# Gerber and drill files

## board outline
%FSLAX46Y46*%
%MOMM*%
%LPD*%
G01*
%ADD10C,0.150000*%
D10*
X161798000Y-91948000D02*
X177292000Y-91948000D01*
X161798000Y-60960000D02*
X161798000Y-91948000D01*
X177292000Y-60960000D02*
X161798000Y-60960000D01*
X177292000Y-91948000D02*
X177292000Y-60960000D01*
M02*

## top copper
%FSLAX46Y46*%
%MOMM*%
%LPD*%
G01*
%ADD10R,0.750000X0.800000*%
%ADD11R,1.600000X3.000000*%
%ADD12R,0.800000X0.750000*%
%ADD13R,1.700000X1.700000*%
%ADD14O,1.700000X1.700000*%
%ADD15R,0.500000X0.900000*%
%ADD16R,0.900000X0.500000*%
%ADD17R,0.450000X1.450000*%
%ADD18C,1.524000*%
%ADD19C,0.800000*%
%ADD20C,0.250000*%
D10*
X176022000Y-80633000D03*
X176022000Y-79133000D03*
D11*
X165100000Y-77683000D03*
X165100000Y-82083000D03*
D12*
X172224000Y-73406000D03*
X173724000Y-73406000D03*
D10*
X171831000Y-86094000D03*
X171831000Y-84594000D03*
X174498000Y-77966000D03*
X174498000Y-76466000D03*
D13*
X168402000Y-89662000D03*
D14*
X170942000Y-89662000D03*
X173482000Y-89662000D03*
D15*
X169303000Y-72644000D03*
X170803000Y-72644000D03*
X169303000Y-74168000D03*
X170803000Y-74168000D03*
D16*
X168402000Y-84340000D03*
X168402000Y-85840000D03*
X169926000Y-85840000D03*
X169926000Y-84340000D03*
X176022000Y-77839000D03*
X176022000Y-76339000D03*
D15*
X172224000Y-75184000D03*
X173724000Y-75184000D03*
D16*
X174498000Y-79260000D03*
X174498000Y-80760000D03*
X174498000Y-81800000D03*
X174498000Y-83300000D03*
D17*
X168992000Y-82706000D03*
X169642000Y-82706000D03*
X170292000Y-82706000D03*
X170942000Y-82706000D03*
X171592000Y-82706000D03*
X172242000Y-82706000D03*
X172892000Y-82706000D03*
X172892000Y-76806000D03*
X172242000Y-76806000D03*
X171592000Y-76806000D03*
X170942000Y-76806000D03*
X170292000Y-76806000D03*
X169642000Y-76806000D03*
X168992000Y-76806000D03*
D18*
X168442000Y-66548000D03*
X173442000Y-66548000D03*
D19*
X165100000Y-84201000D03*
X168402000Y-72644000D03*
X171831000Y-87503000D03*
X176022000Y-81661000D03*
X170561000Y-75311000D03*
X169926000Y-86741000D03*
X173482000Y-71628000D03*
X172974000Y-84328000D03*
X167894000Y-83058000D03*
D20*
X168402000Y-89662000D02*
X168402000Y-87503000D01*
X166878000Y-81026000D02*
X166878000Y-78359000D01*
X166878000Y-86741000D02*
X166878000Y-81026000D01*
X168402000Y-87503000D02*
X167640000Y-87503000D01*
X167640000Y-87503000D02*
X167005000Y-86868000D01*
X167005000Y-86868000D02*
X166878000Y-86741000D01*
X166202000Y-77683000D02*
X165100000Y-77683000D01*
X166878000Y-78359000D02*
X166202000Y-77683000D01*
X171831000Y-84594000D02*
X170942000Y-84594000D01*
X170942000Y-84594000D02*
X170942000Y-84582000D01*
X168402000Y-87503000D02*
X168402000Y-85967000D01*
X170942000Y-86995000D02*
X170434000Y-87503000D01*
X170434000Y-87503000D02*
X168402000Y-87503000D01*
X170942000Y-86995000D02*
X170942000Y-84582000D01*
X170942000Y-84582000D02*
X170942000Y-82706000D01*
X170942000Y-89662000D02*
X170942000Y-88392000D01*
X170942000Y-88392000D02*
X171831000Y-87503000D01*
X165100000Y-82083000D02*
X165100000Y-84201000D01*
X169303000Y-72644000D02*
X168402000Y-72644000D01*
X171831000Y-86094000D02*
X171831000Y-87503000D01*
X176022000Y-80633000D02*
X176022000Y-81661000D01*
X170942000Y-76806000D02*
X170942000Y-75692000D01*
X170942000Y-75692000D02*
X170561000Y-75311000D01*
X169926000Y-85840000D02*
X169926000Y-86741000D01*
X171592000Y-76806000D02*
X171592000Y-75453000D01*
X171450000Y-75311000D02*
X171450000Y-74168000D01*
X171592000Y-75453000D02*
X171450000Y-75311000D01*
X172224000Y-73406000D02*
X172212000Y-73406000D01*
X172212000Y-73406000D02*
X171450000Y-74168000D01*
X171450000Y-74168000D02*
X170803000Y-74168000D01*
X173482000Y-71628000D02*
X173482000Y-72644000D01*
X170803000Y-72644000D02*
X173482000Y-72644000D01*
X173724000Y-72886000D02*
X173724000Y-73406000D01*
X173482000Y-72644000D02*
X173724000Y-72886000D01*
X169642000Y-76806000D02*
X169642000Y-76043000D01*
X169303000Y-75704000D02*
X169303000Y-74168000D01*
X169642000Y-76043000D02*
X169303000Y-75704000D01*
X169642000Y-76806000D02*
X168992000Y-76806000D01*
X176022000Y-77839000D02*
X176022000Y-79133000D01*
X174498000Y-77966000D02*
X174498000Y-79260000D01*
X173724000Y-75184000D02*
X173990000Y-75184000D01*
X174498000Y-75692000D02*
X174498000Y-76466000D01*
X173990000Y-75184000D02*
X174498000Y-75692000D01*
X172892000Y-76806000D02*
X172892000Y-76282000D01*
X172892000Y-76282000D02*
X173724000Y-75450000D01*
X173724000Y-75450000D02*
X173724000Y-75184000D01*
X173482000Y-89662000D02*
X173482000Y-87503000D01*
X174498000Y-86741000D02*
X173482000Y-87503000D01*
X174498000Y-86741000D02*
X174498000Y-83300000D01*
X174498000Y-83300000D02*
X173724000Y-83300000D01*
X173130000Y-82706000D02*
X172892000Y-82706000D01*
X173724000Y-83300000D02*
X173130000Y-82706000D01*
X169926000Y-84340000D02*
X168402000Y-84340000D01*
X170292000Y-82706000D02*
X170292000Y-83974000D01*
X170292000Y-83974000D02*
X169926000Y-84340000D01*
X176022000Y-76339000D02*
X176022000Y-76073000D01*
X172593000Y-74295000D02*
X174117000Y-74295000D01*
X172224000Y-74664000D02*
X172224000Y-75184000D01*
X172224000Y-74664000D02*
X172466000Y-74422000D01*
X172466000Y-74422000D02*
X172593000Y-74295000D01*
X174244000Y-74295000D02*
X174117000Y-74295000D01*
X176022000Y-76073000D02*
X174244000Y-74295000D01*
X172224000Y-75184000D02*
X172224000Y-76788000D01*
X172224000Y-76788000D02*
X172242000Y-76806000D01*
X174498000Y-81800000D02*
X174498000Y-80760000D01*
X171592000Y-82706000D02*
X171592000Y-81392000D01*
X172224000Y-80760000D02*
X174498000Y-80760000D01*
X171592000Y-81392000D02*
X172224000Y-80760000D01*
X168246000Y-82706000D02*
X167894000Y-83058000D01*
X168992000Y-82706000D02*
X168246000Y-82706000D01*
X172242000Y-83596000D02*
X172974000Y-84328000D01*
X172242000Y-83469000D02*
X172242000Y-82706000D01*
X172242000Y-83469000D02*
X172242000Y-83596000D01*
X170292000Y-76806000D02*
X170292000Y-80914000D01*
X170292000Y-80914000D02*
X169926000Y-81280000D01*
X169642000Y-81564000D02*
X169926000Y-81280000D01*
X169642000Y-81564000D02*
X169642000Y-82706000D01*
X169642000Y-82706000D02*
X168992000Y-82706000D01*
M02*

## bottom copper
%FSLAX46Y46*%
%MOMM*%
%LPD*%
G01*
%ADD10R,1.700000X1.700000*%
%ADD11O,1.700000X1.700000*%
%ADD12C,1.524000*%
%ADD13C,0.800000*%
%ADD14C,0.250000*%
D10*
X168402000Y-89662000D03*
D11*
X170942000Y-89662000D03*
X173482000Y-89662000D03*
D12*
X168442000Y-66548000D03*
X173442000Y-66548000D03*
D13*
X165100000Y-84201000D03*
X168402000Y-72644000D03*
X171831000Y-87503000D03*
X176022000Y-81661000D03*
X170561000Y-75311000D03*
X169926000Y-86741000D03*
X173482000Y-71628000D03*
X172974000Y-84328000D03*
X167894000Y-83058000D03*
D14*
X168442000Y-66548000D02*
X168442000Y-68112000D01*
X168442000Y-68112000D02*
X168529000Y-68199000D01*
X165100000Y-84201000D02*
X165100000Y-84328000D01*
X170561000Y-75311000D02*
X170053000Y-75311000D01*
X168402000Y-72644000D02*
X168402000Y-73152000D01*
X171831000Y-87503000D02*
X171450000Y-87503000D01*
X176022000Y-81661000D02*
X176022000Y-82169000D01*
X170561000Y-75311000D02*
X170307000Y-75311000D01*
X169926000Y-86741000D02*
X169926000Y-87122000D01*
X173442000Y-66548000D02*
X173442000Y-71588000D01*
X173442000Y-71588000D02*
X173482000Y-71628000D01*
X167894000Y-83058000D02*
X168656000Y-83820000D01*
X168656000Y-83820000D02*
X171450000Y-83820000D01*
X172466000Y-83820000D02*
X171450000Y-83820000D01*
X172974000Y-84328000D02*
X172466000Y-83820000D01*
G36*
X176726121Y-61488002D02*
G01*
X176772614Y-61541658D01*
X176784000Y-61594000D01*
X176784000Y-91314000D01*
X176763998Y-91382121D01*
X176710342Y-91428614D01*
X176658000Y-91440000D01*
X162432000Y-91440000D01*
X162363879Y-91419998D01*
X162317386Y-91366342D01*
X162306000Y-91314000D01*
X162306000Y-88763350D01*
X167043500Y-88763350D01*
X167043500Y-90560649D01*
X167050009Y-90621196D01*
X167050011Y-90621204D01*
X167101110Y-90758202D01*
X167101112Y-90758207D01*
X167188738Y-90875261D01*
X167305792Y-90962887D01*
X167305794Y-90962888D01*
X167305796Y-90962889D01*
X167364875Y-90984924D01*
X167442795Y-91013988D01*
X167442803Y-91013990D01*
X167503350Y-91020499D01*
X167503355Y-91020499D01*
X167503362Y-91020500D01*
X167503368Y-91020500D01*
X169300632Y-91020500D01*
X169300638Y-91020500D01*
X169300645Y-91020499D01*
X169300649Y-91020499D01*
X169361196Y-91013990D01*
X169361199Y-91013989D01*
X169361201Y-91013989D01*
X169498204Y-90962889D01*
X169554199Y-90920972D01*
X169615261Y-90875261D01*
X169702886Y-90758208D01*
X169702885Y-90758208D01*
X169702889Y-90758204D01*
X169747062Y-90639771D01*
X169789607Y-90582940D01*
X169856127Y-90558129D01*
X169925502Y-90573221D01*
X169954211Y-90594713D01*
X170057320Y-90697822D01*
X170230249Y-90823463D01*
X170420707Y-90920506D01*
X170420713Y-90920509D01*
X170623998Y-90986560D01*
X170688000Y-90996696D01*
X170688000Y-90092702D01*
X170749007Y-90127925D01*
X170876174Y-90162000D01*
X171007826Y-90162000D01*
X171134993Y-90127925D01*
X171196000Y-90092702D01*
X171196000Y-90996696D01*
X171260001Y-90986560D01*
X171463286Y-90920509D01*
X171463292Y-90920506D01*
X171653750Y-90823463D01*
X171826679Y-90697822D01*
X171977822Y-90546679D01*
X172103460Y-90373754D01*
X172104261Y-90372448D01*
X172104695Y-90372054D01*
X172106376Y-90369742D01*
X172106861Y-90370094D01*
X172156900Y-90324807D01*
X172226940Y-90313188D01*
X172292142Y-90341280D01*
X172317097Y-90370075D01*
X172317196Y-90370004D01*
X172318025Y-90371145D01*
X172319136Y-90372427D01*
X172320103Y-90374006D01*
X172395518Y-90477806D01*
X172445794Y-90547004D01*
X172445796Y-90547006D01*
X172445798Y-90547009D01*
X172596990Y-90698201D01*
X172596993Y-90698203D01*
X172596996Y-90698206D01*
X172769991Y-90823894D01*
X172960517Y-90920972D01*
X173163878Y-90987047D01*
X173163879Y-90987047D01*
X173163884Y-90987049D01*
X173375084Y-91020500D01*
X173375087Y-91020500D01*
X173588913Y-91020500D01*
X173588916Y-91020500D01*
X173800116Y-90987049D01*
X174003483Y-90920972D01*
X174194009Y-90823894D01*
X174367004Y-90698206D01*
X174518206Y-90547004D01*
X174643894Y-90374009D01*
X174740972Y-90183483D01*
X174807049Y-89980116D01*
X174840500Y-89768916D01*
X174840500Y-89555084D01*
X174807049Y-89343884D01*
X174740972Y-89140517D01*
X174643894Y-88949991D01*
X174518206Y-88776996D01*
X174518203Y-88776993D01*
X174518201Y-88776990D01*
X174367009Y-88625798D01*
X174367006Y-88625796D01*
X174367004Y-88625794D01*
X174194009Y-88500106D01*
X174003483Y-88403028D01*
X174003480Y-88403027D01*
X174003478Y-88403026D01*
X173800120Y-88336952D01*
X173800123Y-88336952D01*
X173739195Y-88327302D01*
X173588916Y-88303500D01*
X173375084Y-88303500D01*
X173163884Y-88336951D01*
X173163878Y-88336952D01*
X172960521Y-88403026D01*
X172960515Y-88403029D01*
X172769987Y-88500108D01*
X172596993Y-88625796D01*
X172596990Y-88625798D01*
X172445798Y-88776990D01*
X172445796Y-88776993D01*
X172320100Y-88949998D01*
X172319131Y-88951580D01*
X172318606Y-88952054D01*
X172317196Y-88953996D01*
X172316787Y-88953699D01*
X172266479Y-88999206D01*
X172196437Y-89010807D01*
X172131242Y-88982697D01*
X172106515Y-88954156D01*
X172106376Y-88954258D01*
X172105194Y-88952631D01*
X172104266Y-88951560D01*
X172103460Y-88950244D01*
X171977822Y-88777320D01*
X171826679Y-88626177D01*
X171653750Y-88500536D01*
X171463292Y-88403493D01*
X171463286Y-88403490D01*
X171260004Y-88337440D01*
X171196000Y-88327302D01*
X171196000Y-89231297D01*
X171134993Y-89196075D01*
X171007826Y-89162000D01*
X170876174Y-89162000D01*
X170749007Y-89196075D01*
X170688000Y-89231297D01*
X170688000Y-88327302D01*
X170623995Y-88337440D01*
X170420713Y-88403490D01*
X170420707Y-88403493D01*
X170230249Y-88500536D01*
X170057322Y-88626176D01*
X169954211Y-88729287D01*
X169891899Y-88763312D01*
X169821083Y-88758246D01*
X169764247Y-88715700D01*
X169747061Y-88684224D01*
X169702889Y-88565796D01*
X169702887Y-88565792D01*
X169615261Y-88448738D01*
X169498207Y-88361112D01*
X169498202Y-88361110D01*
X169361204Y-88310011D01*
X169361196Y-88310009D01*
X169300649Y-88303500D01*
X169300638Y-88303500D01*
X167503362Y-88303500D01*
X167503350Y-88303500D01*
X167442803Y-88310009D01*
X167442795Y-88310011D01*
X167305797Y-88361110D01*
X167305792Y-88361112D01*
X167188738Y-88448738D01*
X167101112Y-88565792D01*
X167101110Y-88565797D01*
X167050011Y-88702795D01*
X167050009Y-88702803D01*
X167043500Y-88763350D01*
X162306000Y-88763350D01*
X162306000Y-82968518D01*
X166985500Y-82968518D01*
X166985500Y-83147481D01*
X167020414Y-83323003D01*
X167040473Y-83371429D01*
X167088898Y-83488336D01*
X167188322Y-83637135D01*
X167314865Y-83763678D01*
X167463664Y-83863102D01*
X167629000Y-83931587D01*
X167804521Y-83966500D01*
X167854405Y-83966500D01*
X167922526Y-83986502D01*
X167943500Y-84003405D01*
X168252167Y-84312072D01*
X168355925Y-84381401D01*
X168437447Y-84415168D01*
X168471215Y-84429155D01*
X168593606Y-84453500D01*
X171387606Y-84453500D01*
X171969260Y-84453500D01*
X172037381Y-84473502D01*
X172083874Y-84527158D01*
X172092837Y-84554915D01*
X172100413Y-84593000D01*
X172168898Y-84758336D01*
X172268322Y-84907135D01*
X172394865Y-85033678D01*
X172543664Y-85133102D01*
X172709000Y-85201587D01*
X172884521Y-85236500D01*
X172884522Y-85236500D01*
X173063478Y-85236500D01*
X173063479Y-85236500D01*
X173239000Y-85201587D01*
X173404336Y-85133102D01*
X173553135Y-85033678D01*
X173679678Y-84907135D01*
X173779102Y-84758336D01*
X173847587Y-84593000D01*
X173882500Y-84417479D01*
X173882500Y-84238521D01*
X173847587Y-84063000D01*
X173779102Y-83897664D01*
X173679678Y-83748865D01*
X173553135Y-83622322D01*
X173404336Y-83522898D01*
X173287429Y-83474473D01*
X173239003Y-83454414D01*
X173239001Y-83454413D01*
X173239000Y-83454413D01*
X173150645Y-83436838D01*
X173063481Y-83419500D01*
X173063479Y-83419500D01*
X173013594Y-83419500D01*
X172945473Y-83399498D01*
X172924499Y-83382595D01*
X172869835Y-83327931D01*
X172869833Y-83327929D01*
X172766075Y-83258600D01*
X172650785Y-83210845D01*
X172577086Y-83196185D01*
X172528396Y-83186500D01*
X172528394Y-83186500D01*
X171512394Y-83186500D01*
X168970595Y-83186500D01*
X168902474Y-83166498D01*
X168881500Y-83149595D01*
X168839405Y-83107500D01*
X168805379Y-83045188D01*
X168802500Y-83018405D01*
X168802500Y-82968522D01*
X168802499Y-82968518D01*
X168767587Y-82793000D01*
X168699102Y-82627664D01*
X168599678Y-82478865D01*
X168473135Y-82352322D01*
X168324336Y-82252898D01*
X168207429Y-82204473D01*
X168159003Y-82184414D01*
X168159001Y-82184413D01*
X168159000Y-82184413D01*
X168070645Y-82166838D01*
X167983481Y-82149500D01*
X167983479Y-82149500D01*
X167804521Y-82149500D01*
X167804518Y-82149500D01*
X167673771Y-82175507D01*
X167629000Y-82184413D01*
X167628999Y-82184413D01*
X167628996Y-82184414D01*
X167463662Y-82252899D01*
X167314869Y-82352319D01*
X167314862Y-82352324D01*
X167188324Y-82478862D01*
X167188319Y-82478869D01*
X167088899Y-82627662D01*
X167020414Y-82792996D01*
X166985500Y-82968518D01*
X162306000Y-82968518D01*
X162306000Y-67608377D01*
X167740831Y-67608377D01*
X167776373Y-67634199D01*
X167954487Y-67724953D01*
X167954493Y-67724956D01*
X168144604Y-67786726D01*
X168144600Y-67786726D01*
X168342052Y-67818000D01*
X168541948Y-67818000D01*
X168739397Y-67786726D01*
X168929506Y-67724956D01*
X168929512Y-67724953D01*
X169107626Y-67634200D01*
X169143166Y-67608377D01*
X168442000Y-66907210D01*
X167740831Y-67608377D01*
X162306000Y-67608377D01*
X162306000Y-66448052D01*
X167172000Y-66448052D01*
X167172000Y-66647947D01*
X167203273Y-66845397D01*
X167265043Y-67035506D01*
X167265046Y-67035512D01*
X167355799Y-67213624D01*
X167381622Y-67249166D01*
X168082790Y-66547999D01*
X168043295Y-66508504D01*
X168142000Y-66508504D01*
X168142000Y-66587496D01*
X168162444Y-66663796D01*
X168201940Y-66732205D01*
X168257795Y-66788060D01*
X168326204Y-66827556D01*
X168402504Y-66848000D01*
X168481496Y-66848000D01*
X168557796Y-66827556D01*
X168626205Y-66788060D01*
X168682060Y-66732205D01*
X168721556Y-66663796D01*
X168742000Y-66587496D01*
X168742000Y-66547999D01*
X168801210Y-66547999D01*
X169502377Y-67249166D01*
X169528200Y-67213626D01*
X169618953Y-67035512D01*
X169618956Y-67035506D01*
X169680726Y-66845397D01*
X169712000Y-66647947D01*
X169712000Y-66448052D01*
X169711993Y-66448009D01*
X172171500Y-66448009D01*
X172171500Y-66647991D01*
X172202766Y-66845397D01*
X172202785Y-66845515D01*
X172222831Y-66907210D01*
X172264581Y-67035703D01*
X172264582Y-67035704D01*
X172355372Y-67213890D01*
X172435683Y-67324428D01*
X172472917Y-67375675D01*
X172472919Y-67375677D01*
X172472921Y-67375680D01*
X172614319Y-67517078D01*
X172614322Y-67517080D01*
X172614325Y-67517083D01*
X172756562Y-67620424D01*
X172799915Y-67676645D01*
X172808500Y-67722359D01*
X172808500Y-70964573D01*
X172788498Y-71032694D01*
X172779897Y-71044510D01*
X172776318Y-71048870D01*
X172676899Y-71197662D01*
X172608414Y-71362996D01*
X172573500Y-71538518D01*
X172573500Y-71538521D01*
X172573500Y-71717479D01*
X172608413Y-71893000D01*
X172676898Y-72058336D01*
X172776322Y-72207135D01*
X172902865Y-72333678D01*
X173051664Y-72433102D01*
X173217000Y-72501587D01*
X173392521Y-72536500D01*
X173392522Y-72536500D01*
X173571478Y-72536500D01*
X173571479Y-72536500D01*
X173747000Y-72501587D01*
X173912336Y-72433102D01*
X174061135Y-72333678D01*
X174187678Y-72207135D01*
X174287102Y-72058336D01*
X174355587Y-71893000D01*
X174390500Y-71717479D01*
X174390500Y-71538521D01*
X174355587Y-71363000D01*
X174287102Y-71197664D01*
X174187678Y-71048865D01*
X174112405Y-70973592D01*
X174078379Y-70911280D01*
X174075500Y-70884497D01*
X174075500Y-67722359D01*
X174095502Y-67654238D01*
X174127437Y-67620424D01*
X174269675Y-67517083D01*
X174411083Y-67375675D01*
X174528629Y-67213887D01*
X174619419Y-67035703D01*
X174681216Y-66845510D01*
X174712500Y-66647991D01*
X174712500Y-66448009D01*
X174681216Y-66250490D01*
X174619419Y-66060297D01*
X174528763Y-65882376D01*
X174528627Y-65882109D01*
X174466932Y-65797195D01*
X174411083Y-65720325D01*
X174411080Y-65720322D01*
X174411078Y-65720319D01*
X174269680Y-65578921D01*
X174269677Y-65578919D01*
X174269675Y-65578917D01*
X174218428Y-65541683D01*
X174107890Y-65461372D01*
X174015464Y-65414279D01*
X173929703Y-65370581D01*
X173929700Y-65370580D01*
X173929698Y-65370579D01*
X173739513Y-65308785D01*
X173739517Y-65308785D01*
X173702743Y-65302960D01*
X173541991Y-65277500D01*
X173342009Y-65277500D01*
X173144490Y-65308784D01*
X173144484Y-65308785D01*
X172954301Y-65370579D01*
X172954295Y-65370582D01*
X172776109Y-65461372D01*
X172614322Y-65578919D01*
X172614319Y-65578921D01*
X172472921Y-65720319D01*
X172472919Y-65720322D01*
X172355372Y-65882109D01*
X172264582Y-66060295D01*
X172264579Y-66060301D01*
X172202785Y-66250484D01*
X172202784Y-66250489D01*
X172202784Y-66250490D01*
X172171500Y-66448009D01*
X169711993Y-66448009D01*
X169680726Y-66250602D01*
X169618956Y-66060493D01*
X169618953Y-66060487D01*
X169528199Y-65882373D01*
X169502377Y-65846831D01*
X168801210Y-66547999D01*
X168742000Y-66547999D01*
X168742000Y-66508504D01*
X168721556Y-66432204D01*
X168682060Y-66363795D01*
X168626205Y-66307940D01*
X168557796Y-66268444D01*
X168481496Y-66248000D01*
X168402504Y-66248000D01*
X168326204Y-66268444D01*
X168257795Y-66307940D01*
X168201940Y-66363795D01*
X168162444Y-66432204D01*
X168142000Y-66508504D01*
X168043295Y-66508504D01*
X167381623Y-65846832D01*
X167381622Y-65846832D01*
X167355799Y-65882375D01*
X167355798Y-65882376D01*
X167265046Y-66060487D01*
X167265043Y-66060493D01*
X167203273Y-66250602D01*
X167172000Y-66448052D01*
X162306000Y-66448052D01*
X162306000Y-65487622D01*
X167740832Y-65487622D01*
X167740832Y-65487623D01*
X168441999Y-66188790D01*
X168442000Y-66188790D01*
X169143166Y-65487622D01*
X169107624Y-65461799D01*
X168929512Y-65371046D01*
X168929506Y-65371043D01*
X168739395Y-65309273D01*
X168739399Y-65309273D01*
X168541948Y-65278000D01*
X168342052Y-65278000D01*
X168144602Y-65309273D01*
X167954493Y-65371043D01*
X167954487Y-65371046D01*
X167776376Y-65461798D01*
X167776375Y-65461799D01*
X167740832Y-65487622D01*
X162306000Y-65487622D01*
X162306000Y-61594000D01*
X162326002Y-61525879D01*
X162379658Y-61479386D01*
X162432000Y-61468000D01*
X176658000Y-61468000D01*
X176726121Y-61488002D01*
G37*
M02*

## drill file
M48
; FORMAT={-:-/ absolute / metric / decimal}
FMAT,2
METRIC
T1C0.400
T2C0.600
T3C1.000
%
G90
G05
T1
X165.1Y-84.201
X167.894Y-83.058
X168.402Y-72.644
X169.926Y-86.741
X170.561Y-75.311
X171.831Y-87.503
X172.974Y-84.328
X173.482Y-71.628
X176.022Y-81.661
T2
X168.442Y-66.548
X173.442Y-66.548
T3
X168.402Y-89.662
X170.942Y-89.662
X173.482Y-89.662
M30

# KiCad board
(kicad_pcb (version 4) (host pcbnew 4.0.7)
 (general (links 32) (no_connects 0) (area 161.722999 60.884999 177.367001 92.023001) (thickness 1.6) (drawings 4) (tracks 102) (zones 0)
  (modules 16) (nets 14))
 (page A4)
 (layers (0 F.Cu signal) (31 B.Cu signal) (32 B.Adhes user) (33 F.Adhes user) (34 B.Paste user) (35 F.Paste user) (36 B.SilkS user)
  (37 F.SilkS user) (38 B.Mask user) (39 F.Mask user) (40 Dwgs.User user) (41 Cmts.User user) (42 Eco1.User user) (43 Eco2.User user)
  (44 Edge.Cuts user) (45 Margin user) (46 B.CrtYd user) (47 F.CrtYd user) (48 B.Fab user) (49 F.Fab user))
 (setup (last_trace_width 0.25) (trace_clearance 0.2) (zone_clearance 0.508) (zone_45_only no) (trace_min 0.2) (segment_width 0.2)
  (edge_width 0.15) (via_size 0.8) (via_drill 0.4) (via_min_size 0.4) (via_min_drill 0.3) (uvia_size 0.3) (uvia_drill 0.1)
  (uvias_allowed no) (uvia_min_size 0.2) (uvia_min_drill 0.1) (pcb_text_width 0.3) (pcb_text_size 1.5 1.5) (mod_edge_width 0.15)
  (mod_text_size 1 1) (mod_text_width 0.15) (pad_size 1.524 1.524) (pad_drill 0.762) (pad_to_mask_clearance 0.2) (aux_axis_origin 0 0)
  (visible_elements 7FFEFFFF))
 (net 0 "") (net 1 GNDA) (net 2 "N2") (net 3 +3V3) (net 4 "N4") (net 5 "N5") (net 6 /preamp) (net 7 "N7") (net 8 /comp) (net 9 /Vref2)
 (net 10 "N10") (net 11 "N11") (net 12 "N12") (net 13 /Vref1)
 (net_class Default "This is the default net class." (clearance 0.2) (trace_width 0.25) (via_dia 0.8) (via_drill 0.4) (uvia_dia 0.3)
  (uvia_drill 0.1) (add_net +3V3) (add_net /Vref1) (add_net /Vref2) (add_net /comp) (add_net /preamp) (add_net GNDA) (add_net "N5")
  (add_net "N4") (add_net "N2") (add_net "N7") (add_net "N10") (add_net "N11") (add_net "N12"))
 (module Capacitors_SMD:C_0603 (layer F.Cu) (at 176.022 79.883 270)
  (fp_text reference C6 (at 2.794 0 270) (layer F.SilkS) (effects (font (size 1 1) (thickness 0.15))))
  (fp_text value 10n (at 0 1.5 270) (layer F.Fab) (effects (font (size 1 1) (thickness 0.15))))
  (pad 2 smd rect (at 0.75 0 270) (size 0.8 0.75) (layers F.Cu F.Paste F.Mask) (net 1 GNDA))
  (pad 1 smd rect (at -0.75 0 270) (size 0.8 0.75) (layers F.Cu F.Paste F.Mask) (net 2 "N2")))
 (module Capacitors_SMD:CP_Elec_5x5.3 (layer F.Cu) (at 165.1 79.883 270)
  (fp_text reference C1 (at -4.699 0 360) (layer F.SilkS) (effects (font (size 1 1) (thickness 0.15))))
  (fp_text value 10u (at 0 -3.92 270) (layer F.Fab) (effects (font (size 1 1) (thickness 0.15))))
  (pad 1 smd rect (at -2.2 0 90) (size 3 1.6) (layers F.Cu F.Paste F.Mask) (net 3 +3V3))
  (pad 2 smd rect (at 2.2 0 90) (size 3 1.6) (layers F.Cu F.Paste F.Mask) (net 1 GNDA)))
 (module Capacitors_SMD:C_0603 (layer F.Cu) (at 172.974 73.406 180)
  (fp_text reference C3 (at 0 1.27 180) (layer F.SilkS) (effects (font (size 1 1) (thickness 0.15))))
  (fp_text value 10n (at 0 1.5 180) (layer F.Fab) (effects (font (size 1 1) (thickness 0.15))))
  (pad 2 smd rect (at 0.75 0 180) (size 0.8 0.75) (layers F.Cu F.Paste F.Mask) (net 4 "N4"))
  (pad 1 smd rect (at -0.75 0 180) (size 0.8 0.75) (layers F.Cu F.Paste F.Mask) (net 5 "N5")))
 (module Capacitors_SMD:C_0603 (layer F.Cu) (at 171.831 85.344 270)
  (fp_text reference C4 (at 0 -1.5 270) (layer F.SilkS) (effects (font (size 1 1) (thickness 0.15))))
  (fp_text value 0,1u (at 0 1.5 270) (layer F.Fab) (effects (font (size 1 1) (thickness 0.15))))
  (pad 2 smd rect (at 0.75 0 270) (size 0.8 0.75) (layers F.Cu F.Paste F.Mask) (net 1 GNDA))
  (pad 1 smd rect (at -0.75 0 270) (size 0.8 0.75) (layers F.Cu F.Paste F.Mask) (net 3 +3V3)))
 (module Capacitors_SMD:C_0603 (layer F.Cu) (at 174.498 77.216 270)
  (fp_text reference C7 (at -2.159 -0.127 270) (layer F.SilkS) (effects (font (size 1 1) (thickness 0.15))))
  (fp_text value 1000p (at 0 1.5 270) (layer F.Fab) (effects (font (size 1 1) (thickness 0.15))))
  (pad 2 smd rect (at 0.75 0 270) (size 0.8 0.75) (layers F.Cu F.Paste F.Mask) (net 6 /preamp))
  (pad 1 smd rect (at -0.75 0 270) (size 0.8 0.75) (layers F.Cu F.Paste F.Mask) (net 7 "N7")))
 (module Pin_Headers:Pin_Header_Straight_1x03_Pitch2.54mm (layer B.Cu) (at 168.402 89.662 270)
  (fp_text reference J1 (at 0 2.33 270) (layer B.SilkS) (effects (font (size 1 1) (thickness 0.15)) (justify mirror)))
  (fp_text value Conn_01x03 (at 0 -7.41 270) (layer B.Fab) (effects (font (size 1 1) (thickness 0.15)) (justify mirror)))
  (pad 1 thru_hole rect (at 0 0 270) (size 1.7 1.7) (drill 1) (layers *.Cu *.Mask) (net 3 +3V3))
  (pad 2 thru_hole oval (at 0 -2.54 270) (size 1.7 1.7) (drill 1) (layers *.Cu *.Mask) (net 1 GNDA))
  (pad 3 thru_hole oval (at 0 -5.08 270) (size 1.7 1.7) (drill 1) (layers *.Cu *.Mask) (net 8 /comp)))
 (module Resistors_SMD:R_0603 (layer F.Cu) (at 170.053 72.644)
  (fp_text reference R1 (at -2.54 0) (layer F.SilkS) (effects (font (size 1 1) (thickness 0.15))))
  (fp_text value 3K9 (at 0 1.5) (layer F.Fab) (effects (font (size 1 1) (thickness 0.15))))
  (pad 1 smd rect (at -0.75 0) (size 0.5 0.9) (layers F.Cu F.Paste F.Mask) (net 1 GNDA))
  (pad 2 smd rect (at 0.75 0) (size 0.5 0.9) (layers F.Cu F.Paste F.Mask) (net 5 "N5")))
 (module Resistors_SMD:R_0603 (layer F.Cu) (at 170.053 74.168)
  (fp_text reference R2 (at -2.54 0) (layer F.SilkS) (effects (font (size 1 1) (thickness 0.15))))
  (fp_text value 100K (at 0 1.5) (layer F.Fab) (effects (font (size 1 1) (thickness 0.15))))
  (pad 1 smd rect (at -0.75 0) (size 0.5 0.9) (layers F.Cu F.Paste F.Mask) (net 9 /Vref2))
  (pad 2 smd rect (at 0.75 0) (size 0.5 0.9) (layers F.Cu F.Paste F.Mask) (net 4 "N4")))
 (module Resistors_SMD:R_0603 (layer F.Cu) (at 168.402 85.09 270)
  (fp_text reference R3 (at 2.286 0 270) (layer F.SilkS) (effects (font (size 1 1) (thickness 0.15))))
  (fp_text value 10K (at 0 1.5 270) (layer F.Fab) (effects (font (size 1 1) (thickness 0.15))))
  (pad 1 smd rect (at -0.75 0 270) (size 0.5 0.9) (layers F.Cu F.Paste F.Mask) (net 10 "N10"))
  (pad 2 smd rect (at 0.75 0 270) (size 0.5 0.9) (layers F.Cu F.Paste F.Mask) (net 3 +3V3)))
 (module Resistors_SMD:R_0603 (layer F.Cu) (at 169.926 85.09 90)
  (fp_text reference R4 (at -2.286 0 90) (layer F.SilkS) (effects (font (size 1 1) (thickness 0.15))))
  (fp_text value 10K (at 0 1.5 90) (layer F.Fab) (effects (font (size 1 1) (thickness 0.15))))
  (pad 1 smd rect (at -0.75 0 90) (size 0.5 0.9) (layers F.Cu F.Paste F.Mask) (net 1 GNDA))
  (pad 2 smd rect (at 0.75 0 90) (size 0.5 0.9) (layers F.Cu F.Paste F.Mask) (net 10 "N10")))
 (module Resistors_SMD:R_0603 (layer F.Cu) (at 176.022 77.089 90)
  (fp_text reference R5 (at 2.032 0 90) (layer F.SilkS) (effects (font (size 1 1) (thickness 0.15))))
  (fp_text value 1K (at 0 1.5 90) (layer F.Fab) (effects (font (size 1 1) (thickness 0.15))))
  (pad 1 smd rect (at -0.75 0 90) (size 0.5 0.9) (layers F.Cu F.Paste F.Mask) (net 2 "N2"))
  (pad 2 smd rect (at 0.75 0 90) (size 0.5 0.9) (layers F.Cu F.Paste F.Mask) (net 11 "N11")))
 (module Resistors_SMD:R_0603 (layer F.Cu) (at 172.974 75.184)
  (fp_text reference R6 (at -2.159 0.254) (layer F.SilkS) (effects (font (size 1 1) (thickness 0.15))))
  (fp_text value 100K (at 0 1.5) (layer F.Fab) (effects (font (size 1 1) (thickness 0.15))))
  (pad 1 smd rect (at -0.75 0) (size 0.5 0.9) (layers F.Cu F.Paste F.Mask) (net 11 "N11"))
  (pad 2 smd rect (at 0.75 0) (size 0.5 0.9) (layers F.Cu F.Paste F.Mask) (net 7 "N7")))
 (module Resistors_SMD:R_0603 (layer F.Cu) (at 174.498 80.01 270)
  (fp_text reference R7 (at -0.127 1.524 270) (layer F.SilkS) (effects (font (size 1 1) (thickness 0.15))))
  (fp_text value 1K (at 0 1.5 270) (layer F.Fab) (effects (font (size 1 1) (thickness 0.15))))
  (pad 1 smd rect (at -0.75 0 270) (size 0.5 0.9) (layers F.Cu F.Paste F.Mask) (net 6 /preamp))
  (pad 2 smd rect (at 0.75 0 270) (size 0.5 0.9) (layers F.Cu F.Paste F.Mask) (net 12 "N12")))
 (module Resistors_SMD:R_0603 (layer F.Cu) (at 174.498 82.55 270)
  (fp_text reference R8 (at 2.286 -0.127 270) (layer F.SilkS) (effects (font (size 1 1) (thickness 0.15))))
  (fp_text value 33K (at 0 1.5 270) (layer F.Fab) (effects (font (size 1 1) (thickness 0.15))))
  (pad 1 smd rect (at -0.75 0 270) (size 0.5 0.9) (layers F.Cu F.Paste F.Mask) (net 12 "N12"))
  (pad 2 smd rect (at 0.75 0 270) (size 0.5 0.9) (layers F.Cu F.Paste F.Mask) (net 8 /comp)))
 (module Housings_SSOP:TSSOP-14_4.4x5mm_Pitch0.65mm (layer F.Cu) (at 170.942 79.756 90)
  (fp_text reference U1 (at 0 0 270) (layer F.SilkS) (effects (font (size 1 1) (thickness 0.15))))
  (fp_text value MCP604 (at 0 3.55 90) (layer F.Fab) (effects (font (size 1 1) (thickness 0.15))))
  (pad 1 smd rect (at -2.95 -1.95 90) (size 1.45 0.45) (layers F.Cu F.Paste F.Mask) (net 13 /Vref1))
  (pad 2 smd rect (at -2.95 -1.3 90) (size 1.45 0.45) (layers F.Cu F.Paste F.Mask) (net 13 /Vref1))
  (pad 3 smd rect (at -2.95 -0.65 90) (size 1.45 0.45) (layers F.Cu F.Paste F.Mask) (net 10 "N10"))
  (pad 4 smd rect (at -2.95 0 90) (size 1.45 0.45) (layers F.Cu F.Paste F.Mask) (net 3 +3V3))
  (pad 5 smd rect (at -2.95 0.65 90) (size 1.45 0.45) (layers F.Cu F.Paste F.Mask) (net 12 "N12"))
  (pad 6 smd rect (at -2.95 1.3 90) (size 1.45 0.45) (layers F.Cu F.Paste F.Mask) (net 13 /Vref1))
  (pad 7 smd rect (at -2.95 1.95 90) (size 1.45 0.45) (layers F.Cu F.Paste F.Mask) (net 8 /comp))
  (pad 8 smd rect (at 2.95 1.95 90) (size 1.45 0.45) (layers F.Cu F.Paste F.Mask) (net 7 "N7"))
  (pad 9 smd rect (at 2.95 1.3 90) (size 1.45 0.45) (layers F.Cu F.Paste F.Mask) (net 11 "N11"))
  (pad 10 smd rect (at 2.95 0.65 90) (size 1.45 0.45) (layers F.Cu F.Paste F.Mask) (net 4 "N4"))
  (pad 11 smd rect (at 2.95 0 90) (size 1.45 0.45) (layers F.Cu F.Paste F.Mask) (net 1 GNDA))
  (pad 12 smd rect (at 2.95 -0.65 90) (size 1.45 0.45) (layers F.Cu F.Paste F.Mask) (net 13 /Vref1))
  (pad 13 smd rect (at 2.95 -1.3 90) (size 1.45 0.45) (layers F.Cu F.Paste F.Mask) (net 9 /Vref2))
  (pad 14 smd rect (at 2.95 -1.95 90) (size 1.45 0.45) (layers F.Cu F.Paste F.Mask) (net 9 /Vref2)))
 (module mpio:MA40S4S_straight (layer F.Cu) (at 170.942 66.548)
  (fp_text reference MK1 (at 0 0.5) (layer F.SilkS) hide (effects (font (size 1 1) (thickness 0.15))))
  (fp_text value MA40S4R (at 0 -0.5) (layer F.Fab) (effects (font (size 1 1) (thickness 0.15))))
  (pad 1 thru_hole circle (at -2.5 0) (size 1.524 1.524) (drill 0.6) (layers *.Cu *.Mask) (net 1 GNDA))
  (pad 2 thru_hole circle (at 2.5 0) (size 1.524 1.524) (drill 0.6) (layers *.Cu *.Mask) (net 5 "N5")))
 (gr_line (start 161.798 91.948) (end 177.292 91.948) (angle 90) (layer Edge.Cuts) (width 0.15))
 (gr_line (start 161.798 60.96) (end 161.798 91.948) (angle 90) (layer Edge.Cuts) (width 0.15))
 (gr_line (start 177.292 60.96) (end 161.798 60.96) (angle 90) (layer Edge.Cuts) (width 0.15))
 (gr_line (start 177.292 91.948) (end 177.292 60.96) (angle 90) (layer Edge.Cuts) (width 0.15))
 (segment (start 168.402 89.662) (end 168.402 87.503) (width 0.25) (layer F.Cu) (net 3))
 (segment (start 166.878 81.026) (end 166.878 78.359) (width 0.25) (layer F.Cu) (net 3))
 (segment (start 166.878 86.741) (end 166.878 81.026) (width 0.25) (layer F.Cu) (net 3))
 (segment (start 168.402 87.503) (end 167.64 87.503) (width 0.25) (layer F.Cu) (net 3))
 (segment (start 167.64 87.503) (end 167.005 86.868) (width 0.25) (layer F.Cu) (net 3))
 (segment (start 167.005 86.868) (end 166.878 86.741) (width 0.25) (layer F.Cu) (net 3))
 (segment (start 166.202 77.683) (end 165.1 77.683) (width 0.25) (layer F.Cu) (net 3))
 (segment (start 166.878 78.359) (end 166.202 77.683) (width 0.25) (layer F.Cu) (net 3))
 (segment (start 171.831 84.594) (end 170.942 84.594) (width 0.25) (layer F.Cu) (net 3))
 (segment (start 170.942 84.594) (end 170.942 84.582) (width 0.25) (layer F.Cu) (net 3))
 (segment (start 168.402 87.503) (end 168.402 85.967) (width 0.25) (layer F.Cu) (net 3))
 (segment (start 170.942 86.995) (end 170.434 87.503) (width 0.25) (layer F.Cu) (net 3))
 (segment (start 170.434 87.503) (end 168.402 87.503) (width 0.25) (layer F.Cu) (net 3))
 (segment (start 170.942 86.995) (end 170.942 84.582) (width 0.25) (layer F.Cu) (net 3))
 (segment (start 170.942 84.582) (end 170.942 82.706) (width 0.25) (layer F.Cu) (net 3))
 (segment (start 170.942 89.662) (end 170.942 88.392) (width 0.25) (layer F.Cu) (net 1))
 (segment (start 170.942 88.392) (end 171.831 87.503) (width 0.25) (layer F.Cu) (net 1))
 (segment (start 168.442 66.548) (end 168.442 68.112) (width 0.25) (layer B.Cu) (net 1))
 (segment (start 168.442 68.112) (end 168.529 68.199) (width 0.25) (layer B.Cu) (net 1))
 (segment (start 165.1 82.083) (end 165.1 84.201) (width 0.25) (layer F.Cu) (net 1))
 (segment (start 165.1 84.201) (end 165.1 84.328) (width 0.25) (layer B.Cu) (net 1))
 (via (at 165.1 84.201) (size 0.8) (drill 0.4) (layers F.Cu B.Cu) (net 1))
 (segment (start 170.561 75.311) (end 170.053 75.311) (width 0.25) (layer B.Cu) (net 1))
 (segment (start 169.303 72.644) (end 168.402 72.644) (width 0.25) (layer F.Cu) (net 1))
 (segment (start 168.402 72.644) (end 168.402 73.152) (width 0.25) (layer B.Cu) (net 1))
 (via (at 168.402 72.644) (size 0.8) (drill 0.4) (layers F.Cu B.Cu) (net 1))
 (segment (start 171.831 86.094) (end 171.831 87.503) (width 0.25) (layer F.Cu) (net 1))
 (segment (start 171.831 87.503) (end 171.45 87.503) (width 0.25) (layer B.Cu) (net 1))
 (via (at 171.831 87.503) (size 0.8) (drill 0.4) (layers F.Cu B.Cu) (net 1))
 (segment (start 176.022 80.633) (end 176.022 81.661) (width 0.25) (layer F.Cu) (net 1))
 (segment (start 176.022 81.661) (end 176.022 82.169) (width 0.25) (layer B.Cu) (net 1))
 (via (at 176.022 81.661) (size 0.8) (drill 0.4) (layers F.Cu B.Cu) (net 1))
 (segment (start 170.942 76.806) (end 170.942 75.692) (width 0.25) (layer F.Cu) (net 1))
 (segment (start 170.561 75.311) (end 170.307 75.311) (width 0.25) (layer B.Cu) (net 1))
 (via (at 170.561 75.311) (size 0.8) (drill 0.4) (layers F.Cu B.Cu) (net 1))
 (segment (start 170.942 75.692) (end 170.561 75.311) (width 0.25) (layer F.Cu) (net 1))
 (segment (start 169.926 85.84) (end 169.926 86.741) (width 0.25) (layer F.Cu) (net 1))
 (segment (start 169.926 86.741) (end 169.926 87.122) (width 0.25) (layer B.Cu) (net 1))
 (via (at 169.926 86.741) (size 0.8) (drill 0.4) (layers F.Cu B.Cu) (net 1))
 (segment (start 171.592 76.806) (end 171.592 75.453) (width 0.25) (layer F.Cu) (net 4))
 (segment (start 171.45 75.311) (end 171.45 74.168) (width 0.25) (layer F.Cu) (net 4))
 (segment (start 171.592 75.453) (end 171.45 75.311) (width 0.25) (layer F.Cu) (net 4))
 (segment (start 172.224 73.406) (end 172.212 73.406) (width 0.25) (layer F.Cu) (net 4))
 (segment (start 172.212 73.406) (end 171.45 74.168) (width 0.25) (layer F.Cu) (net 4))
 (segment (start 171.45 74.168) (end 170.803 74.168) (width 0.25) (layer F.Cu) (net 4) (status 20))
 (segment (start 173.442 66.548) (end 173.442 71.588) (width 0.25) (layer B.Cu) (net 5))
 (segment (start 173.482 71.628) (end 173.482 72.644) (width 0.25) (layer F.Cu) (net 5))
 (via (at 173.482 71.628) (size 0.8) (drill 0.4) (layers F.Cu B.Cu) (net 5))
 (segment (start 173.442 71.588) (end 173.482 71.628) (width 0.25) (layer B.Cu) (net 5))
 (segment (start 170.803 72.644) (end 173.482 72.644) (width 0.25) (layer F.Cu) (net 5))
 (segment (start 173.724 72.886) (end 173.724 73.406) (width 0.25) (layer F.Cu) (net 5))
 (segment (start 173.482 72.644) (end 173.724 72.886) (width 0.25) (layer F.Cu) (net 5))
 (segment (start 169.642 76.806) (end 169.642 76.043) (width 0.25) (layer F.Cu) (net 9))
 (segment (start 169.303 75.704) (end 169.303 74.168) (width 0.25) (layer F.Cu) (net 9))
 (segment (start 169.642 76.043) (end 169.303 75.704) (width 0.25) (layer F.Cu) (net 9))
 (segment (start 169.642 76.806) (end 168.992 76.806) (width 0.25) (layer F.Cu) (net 9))
 (segment (start 176.022 77.839) (end 176.022 79.133) (width 0.25) (layer F.Cu) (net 2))
 (segment (start 174.498 77.966) (end 174.498 79.26) (width 0.25) (layer F.Cu) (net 6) (status 20))
 (segment (start 173.724 75.184) (end 173.99 75.184) (width 0.25) (layer F.Cu) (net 7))
 (segment (start 174.498 75.692) (end 174.498 76.466) (width 0.25) (layer F.Cu) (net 7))
 (segment (start 173.99 75.184) (end 174.498 75.692) (width 0.25) (layer F.Cu) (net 7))
 (segment (start 172.892 76.806) (end 172.892 76.282) (width 0.25) (layer F.Cu) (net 7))
 (segment (start 172.892 76.282) (end 173.724 75.45) (width 0.25) (layer F.Cu) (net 7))
 (segment (start 173.724 75.45) (end 173.724 75.184) (width 0.25) (layer F.Cu) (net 7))
 (segment (start 173.482 89.662) (end 173.482 87.503) (width 0.25) (layer F.Cu) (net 8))
 (segment (start 174.498 86.741) (end 173.482 87.503) (width 0.25) (layer F.Cu) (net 8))
 (segment (start 174.498 86.741) (end 174.498 83.3) (width 0.25) (layer F.Cu) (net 8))
 (segment (start 174.498 83.3) (end 173.724 83.3) (width 0.25) (layer F.Cu) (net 8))
 (segment (start 173.13 82.706) (end 172.892 82.706) (width 0.25) (layer F.Cu) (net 8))
 (segment (start 173.724 83.3) (end 173.13 82.706) (width 0.25) (layer F.Cu) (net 8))
 (segment (start 169.926 84.34) (end 168.402 84.34) (width 0.25) (layer F.Cu) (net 10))
 (segment (start 170.292 82.706) (end 170.292 83.974) (width 0.25) (layer F.Cu) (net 10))
 (segment (start 170.292 83.974) (end 169.926 84.34) (width 0.25) (layer F.Cu) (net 10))
 (segment (start 176.022 76.339) (end 176.022 76.073) (width 0.25) (layer F.Cu) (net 11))
 (segment (start 172.593 74.295) (end 174.117 74.295) (width 0.25) (layer F.Cu) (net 11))
 (segment (start 172.224 74.664) (end 172.224 75.184) (width 0.25) (layer F.Cu) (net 11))
 (segment (start 172.224 74.664) (end 172.466 74.422) (width 0.25) (layer F.Cu) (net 11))
 (segment (start 172.466 74.422) (end 172.593 74.295) (width 0.25) (layer F.Cu) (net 11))
 (segment (start 174.244 74.295) (end 174.117 74.295) (width 0.25) (layer F.Cu) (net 11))
 (segment (start 176.022 76.073) (end 174.244 74.295) (width 0.25) (layer F.Cu) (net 11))
 (segment (start 172.224 75.184) (end 172.224 76.788) (width 0.25) (layer F.Cu) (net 11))
 (segment (start 172.224 76.788) (end 172.242 76.806) (width 0.25) (layer F.Cu) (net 11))
 (segment (start 174.498 81.8) (end 174.498 80.76) (width 0.25) (layer F.Cu) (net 12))
 (segment (start 171.592 82.706) (end 171.592 81.392) (width 0.25) (layer F.Cu) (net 12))
 (segment (start 172.224 80.76) (end 174.498 80.76) (width 0.25) (layer F.Cu) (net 12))
 (segment (start 171.592 81.392) (end 172.224 80.76) (width 0.25) (layer F.Cu) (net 12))
 (via (at 172.974 84.328) (size 0.8) (drill 0.4) (layers F.Cu B.Cu) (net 13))
 (segment (start 168.246 82.706) (end 167.894 83.058) (width 0.25) (layer F.Cu) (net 13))
 (via (at 167.894 83.058) (size 0.8) (drill 0.4) (layers F.Cu B.Cu) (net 13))
 (segment (start 167.894 83.058) (end 168.656 83.82) (width 0.25) (layer B.Cu) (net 13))
 (segment (start 168.656 83.82) (end 171.45 83.82) (width 0.25) (layer B.Cu) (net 13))
 (segment (start 168.992 82.706) (end 168.246 82.706) (width 0.25) (layer F.Cu) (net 13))
 (segment (start 172.242 83.596) (end 172.974 84.328) (width 0.25) (layer F.Cu) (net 13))
 (segment (start 172.242 83.469) (end 172.242 82.706) (width 0.25) (layer F.Cu) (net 13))
 (segment (start 172.242 83.469) (end 172.242 83.596) (width 0.25) (layer F.Cu) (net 13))
 (segment (start 172.466 83.82) (end 171.45 83.82) (width 0.25) (layer B.Cu) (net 13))
 (segment (start 172.974 84.328) (end 172.466 83.82) (width 0.25) (layer B.Cu) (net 13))
 (segment (start 170.292 76.806) (end 170.292 80.914) (width 0.25) (layer F.Cu) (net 13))
 (segment (start 170.292 80.914) (end 169.926 81.28) (width 0.25) (layer F.Cu) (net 13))
 (segment (start 169.642 81.564) (end 169.926 81.28) (width 0.25) (layer F.Cu) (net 13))
 (segment (start 169.642 81.564) (end 169.642 82.706) (width 0.25) (layer F.Cu) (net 13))
 (segment (start 169.642 82.706) (end 168.992 82.706) (width 0.25) (layer F.Cu) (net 13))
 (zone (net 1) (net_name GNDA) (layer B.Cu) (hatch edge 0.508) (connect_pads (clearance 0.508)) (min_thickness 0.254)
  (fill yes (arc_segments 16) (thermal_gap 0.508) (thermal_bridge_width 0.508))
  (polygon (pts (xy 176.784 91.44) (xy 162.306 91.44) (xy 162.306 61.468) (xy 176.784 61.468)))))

